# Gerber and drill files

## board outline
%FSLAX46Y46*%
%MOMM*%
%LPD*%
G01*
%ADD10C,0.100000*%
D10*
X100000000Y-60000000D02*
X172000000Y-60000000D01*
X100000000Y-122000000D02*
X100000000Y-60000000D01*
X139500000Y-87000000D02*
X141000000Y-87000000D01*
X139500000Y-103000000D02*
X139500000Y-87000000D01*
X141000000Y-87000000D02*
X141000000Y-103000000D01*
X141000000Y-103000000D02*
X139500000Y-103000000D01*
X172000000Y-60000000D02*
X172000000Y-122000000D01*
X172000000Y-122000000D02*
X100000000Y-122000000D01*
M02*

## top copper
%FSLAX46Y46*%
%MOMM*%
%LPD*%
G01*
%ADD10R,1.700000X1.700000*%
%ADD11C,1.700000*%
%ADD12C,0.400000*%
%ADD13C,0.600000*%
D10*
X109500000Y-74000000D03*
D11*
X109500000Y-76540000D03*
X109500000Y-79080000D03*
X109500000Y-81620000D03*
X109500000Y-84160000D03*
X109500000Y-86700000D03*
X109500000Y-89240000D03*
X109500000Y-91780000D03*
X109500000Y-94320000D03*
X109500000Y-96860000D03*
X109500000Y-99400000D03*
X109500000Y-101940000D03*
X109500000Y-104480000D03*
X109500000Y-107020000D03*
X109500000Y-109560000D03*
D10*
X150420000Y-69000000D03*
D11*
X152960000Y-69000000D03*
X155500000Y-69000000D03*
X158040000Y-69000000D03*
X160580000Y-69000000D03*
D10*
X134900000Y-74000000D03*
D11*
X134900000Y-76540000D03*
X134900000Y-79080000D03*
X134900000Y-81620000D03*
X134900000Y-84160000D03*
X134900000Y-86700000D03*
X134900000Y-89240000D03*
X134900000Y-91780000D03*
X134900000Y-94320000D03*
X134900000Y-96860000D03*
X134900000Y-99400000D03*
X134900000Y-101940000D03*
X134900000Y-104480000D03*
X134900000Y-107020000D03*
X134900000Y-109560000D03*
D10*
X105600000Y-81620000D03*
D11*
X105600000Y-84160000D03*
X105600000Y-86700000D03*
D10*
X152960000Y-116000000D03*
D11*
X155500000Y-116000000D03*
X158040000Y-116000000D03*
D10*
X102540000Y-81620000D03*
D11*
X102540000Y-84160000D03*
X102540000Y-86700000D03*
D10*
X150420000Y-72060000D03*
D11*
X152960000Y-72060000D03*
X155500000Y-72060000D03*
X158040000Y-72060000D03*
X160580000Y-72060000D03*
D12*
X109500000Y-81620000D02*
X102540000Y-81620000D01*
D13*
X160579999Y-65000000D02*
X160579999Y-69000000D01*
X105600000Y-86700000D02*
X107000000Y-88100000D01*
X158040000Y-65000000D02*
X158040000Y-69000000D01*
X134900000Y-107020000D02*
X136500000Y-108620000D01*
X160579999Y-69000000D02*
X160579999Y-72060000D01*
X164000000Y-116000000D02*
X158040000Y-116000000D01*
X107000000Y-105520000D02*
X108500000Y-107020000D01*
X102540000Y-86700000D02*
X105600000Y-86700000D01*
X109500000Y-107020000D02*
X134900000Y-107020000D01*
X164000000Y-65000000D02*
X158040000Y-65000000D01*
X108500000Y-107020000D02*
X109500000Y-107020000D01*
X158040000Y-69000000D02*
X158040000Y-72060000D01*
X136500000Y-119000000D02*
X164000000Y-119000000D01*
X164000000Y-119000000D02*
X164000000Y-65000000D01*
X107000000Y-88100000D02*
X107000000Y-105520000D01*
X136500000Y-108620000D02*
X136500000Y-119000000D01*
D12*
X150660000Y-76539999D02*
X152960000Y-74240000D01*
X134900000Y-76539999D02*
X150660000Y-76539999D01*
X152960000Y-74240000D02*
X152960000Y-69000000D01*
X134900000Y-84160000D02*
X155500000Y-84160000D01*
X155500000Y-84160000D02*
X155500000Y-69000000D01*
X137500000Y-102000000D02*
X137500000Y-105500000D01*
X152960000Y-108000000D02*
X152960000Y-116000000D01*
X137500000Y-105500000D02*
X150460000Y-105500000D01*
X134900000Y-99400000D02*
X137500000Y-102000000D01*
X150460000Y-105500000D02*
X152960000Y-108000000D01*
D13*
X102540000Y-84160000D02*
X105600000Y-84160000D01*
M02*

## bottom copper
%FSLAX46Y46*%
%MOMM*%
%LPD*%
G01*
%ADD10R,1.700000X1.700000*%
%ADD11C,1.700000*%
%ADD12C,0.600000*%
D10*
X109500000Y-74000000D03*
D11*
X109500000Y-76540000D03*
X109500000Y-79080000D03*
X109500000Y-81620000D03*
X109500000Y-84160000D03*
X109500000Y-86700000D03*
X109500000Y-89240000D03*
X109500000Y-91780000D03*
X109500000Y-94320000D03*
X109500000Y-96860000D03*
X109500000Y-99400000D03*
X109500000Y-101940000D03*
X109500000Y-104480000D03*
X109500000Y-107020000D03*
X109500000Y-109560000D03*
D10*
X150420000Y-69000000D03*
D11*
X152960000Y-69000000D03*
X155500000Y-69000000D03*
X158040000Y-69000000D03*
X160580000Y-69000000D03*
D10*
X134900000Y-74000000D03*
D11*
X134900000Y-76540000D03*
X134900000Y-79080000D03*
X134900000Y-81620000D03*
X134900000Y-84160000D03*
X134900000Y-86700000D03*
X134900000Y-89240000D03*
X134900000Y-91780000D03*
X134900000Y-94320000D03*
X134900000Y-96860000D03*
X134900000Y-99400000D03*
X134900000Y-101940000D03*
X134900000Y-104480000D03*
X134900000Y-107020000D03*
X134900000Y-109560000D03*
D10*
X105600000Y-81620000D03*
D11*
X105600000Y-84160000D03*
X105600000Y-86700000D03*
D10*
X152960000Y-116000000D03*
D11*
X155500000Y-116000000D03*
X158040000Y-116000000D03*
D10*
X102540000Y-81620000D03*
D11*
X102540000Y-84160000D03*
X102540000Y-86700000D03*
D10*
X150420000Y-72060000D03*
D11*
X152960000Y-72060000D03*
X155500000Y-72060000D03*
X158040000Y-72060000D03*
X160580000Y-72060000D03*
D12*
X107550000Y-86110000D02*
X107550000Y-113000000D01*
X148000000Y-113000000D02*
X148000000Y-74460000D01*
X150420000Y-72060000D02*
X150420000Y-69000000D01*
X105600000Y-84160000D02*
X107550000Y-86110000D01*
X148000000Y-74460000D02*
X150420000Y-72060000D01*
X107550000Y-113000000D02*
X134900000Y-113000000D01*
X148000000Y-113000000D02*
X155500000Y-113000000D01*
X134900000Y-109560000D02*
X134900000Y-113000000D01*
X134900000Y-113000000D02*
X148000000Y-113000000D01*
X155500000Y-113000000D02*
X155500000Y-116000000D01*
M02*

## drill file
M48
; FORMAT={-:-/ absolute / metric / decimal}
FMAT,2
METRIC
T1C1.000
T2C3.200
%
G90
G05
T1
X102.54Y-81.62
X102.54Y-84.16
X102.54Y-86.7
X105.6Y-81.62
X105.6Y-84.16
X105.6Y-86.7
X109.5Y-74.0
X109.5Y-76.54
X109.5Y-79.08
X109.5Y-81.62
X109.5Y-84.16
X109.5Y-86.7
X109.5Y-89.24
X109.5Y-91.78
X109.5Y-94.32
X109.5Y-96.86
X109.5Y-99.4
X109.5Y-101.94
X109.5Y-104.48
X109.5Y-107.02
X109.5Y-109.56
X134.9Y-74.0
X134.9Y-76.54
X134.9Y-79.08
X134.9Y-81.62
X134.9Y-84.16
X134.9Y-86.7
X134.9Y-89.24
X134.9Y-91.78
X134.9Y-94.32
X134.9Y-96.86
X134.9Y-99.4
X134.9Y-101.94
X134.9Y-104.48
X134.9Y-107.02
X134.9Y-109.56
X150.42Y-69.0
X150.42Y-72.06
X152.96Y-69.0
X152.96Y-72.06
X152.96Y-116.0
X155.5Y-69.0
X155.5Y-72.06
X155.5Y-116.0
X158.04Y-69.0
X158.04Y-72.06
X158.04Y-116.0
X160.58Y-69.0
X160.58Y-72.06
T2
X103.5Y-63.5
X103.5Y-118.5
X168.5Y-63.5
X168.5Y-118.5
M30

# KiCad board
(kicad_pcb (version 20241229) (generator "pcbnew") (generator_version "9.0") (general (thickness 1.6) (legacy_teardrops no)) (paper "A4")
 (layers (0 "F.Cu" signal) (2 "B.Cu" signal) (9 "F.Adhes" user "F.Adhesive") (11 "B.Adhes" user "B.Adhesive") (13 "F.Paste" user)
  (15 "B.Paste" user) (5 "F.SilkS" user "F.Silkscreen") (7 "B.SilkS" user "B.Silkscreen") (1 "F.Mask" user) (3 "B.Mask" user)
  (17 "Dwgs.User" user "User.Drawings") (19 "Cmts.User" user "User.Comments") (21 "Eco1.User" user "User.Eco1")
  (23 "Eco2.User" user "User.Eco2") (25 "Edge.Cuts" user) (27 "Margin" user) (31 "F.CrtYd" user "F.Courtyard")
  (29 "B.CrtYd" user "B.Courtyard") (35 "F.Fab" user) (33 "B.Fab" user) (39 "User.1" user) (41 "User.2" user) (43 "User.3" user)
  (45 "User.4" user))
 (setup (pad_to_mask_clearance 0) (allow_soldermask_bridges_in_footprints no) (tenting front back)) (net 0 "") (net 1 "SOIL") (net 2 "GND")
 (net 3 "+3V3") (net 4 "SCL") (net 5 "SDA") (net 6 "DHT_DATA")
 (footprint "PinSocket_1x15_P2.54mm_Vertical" (layer "F.Cu") (at 109.5 74)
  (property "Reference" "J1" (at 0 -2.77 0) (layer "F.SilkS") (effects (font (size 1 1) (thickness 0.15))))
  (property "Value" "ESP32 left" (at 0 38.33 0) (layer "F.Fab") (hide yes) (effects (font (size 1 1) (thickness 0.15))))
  (pad "1" thru_hole rect (at 0 0) (size 1.7 1.7) (drill 1) (layers "*.Cu" "*.Mask") (remove_unused_layers no))
  (pad "2" thru_hole circle (at 0 2.54) (size 1.7 1.7) (drill 1) (layers "*.Cu" "*.Mask") (remove_unused_layers no))
  (pad "3" thru_hole circle (at 0 5.08) (size 1.7 1.7) (drill 1) (layers "*.Cu" "*.Mask") (remove_unused_layers no))
  (pad "4" thru_hole circle (at 0 7.62) (size 1.7 1.7) (drill 1) (layers "*.Cu" "*.Mask") (remove_unused_layers no) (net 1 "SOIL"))
  (pad "5" thru_hole circle (at 0 10.16) (size 1.7 1.7) (drill 1) (layers "*.Cu" "*.Mask") (remove_unused_layers no))
  (pad "6" thru_hole circle (at 0 12.7) (size 1.7 1.7) (drill 1) (layers "*.Cu" "*.Mask") (remove_unused_layers no))
  (pad "7" thru_hole circle (at 0 15.24) (size 1.7 1.7) (drill 1) (layers "*.Cu" "*.Mask") (remove_unused_layers no))
  (pad "8" thru_hole circle (at 0 17.78) (size 1.7 1.7) (drill 1) (layers "*.Cu" "*.Mask") (remove_unused_layers no))
  (pad "9" thru_hole circle (at 0 20.32) (size 1.7 1.7) (drill 1) (layers "*.Cu" "*.Mask") (remove_unused_layers no))
  (pad "10" thru_hole circle (at 0 22.86) (size 1.7 1.7) (drill 1) (layers "*.Cu" "*.Mask") (remove_unused_layers no))
  (pad "11" thru_hole circle (at 0 25.4) (size 1.7 1.7) (drill 1) (layers "*.Cu" "*.Mask") (remove_unused_layers no))
  (pad "12" thru_hole circle (at 0 27.94) (size 1.7 1.7) (drill 1) (layers "*.Cu" "*.Mask") (remove_unused_layers no))
  (pad "13" thru_hole circle (at 0 30.48) (size 1.7 1.7) (drill 1) (layers "*.Cu" "*.Mask") (remove_unused_layers no))
  (pad "14" thru_hole circle (at 0 33.02) (size 1.7 1.7) (drill 1) (layers "*.Cu" "*.Mask") (remove_unused_layers no) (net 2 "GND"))
  (pad "15" thru_hole circle (at 0 35.56) (size 1.7 1.7) (drill 1) (layers "*.Cu" "*.Mask") (remove_unused_layers no)))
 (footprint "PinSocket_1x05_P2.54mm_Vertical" (layer "F.Cu") (at 150.42 69 90)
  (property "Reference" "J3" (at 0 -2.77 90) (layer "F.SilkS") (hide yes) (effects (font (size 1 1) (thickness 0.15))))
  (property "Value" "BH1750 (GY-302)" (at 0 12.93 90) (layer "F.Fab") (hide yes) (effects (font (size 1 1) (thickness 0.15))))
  (pad "1" thru_hole rect (at 0 0 90) (size 1.7 1.7) (drill 1) (layers "*.Cu" "*.Mask") (remove_unused_layers no) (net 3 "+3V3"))
  (pad "2" thru_hole circle (at 0 2.54 90) (size 1.7 1.7) (drill 1) (layers "*.Cu" "*.Mask") (remove_unused_layers no) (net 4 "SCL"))
  (pad "3" thru_hole circle (at 0 5.08 90) (size 1.7 1.7) (drill 1) (layers "*.Cu" "*.Mask") (remove_unused_layers no) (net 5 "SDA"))
  (pad "4" thru_hole circle (at 0 7.62 90) (size 1.7 1.7) (drill 1) (layers "*.Cu" "*.Mask") (remove_unused_layers no) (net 2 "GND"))
  (pad "5" thru_hole circle (at 0 10.16 90) (size 1.7 1.7) (drill 1) (layers "*.Cu" "*.Mask") (remove_unused_layers no) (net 2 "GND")))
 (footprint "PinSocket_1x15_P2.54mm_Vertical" (layer "F.Cu") (at 134.9 74)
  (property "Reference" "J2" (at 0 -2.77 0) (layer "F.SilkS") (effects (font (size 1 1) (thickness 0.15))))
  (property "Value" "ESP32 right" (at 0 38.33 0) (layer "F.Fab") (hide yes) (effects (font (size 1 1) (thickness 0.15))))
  (pad "1" thru_hole rect (at 0 0) (size 1.7 1.7) (drill 1) (layers "*.Cu" "*.Mask") (remove_unused_layers no))
  (pad "2" thru_hole circle (at 0 2.54) (size 1.7 1.7) (drill 1) (layers "*.Cu" "*.Mask") (remove_unused_layers no) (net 4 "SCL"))
  (pad "3" thru_hole circle (at 0 5.08) (size 1.7 1.7) (drill 1) (layers "*.Cu" "*.Mask") (remove_unused_layers no))
  (pad "4" thru_hole circle (at 0 7.62) (size 1.7 1.7) (drill 1) (layers "*.Cu" "*.Mask") (remove_unused_layers no))
  (pad "5" thru_hole circle (at 0 10.16) (size 1.7 1.7) (drill 1) (layers "*.Cu" "*.Mask") (remove_unused_layers no) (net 5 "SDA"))
  (pad "6" thru_hole circle (at 0 12.7) (size 1.7 1.7) (drill 1) (layers "*.Cu" "*.Mask") (remove_unused_layers no))
  (pad "7" thru_hole circle (at 0 15.24) (size 1.7 1.7) (drill 1) (layers "*.Cu" "*.Mask") (remove_unused_layers no))
  (pad "8" thru_hole circle (at 0 17.78) (size 1.7 1.7) (drill 1) (layers "*.Cu" "*.Mask") (remove_unused_layers no))
  (pad "9" thru_hole circle (at 0 20.32) (size 1.7 1.7) (drill 1) (layers "*.Cu" "*.Mask") (remove_unused_layers no))
  (pad "10" thru_hole circle (at 0 22.86) (size 1.7 1.7) (drill 1) (layers "*.Cu" "*.Mask") (remove_unused_layers no))
  (pad "11" thru_hole circle (at 0 25.4) (size 1.7 1.7) (drill 1) (layers "*.Cu" "*.Mask") (remove_unused_layers no) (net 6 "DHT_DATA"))
  (pad "12" thru_hole circle (at 0 27.94) (size 1.7 1.7) (drill 1) (layers "*.Cu" "*.Mask") (remove_unused_layers no))
  (pad "13" thru_hole circle (at 0 30.48) (size 1.7 1.7) (drill 1) (layers "*.Cu" "*.Mask") (remove_unused_layers no))
  (pad "14" thru_hole circle (at 0 33.02) (size 1.7 1.7) (drill 1) (layers "*.Cu" "*.Mask") (remove_unused_layers no) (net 2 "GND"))
  (pad "15" thru_hole circle (at 0 35.56) (size 1.7 1.7) (drill 1) (layers "*.Cu" "*.Mask") (remove_unused_layers no) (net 3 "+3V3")))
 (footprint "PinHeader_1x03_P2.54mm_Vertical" (layer "F.Cu") (at 105.6 81.62)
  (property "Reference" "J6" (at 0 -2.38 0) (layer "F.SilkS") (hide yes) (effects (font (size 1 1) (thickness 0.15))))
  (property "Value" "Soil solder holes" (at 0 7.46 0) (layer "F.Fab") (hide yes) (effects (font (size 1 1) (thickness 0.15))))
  (pad "1" thru_hole rect (at 0 0) (size 1.7 1.7) (drill 1) (layers "*.Cu" "*.Mask") (remove_unused_layers no) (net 1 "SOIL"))
  (pad "2" thru_hole circle (at 0 2.54) (size 1.7 1.7) (drill 1) (layers "*.Cu" "*.Mask") (remove_unused_layers no) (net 3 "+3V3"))
  (pad "3" thru_hole circle (at 0 5.08) (size 1.7 1.7) (drill 1) (layers "*.Cu" "*.Mask") (remove_unused_layers no) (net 2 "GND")))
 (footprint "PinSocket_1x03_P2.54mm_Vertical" (layer "F.Cu") (at 152.96 116 90)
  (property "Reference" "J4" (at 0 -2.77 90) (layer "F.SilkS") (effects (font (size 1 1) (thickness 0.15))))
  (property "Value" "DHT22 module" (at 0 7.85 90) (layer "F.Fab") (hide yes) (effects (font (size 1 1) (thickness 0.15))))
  (pad "1" thru_hole rect (at 0 0 90) (size 1.7 1.7) (drill 1) (layers "*.Cu" "*.Mask") (remove_unused_layers no) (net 6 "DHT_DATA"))
  (pad "2" thru_hole circle (at 0 2.54 90) (size 1.7 1.7) (drill 1) (layers "*.Cu" "*.Mask") (remove_unused_layers no) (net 3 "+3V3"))
  (pad "3" thru_hole circle (at 0 5.08 90) (size 1.7 1.7) (drill 1) (layers "*.Cu" "*.Mask") (remove_unused_layers no) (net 2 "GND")))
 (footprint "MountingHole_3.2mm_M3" (layer "F.Cu") (at 103.5 118.5)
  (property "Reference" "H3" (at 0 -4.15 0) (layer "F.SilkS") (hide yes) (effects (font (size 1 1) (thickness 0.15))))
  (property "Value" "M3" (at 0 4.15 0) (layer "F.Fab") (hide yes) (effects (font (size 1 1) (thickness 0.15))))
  (pad "" np_thru_hole circle (at 0 0) (size 3.2 3.2) (drill 3.2) (layers "*.Cu" "*.Mask")))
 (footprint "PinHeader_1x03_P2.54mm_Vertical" (layer "F.Cu") (at 102.54 81.62)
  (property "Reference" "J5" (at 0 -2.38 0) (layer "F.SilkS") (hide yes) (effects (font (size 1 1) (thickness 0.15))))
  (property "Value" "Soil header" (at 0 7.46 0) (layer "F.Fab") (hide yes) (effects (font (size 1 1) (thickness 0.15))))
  (pad "1" thru_hole rect (at 0 0) (size 1.7 1.7) (drill 1) (layers "*.Cu" "*.Mask") (remove_unused_layers no) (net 1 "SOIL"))
  (pad "2" thru_hole circle (at 0 2.54) (size 1.7 1.7) (drill 1) (layers "*.Cu" "*.Mask") (remove_unused_layers no) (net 3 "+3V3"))
  (pad "3" thru_hole circle (at 0 5.08) (size 1.7 1.7) (drill 1) (layers "*.Cu" "*.Mask") (remove_unused_layers no) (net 2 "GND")))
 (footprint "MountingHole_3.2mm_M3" (layer "F.Cu") (at 168.5 118.5)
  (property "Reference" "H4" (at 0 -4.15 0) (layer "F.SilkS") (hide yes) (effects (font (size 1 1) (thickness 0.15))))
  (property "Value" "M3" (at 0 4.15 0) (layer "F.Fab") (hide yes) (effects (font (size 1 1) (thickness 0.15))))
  (pad "" np_thru_hole circle (at 0 0) (size 3.2 3.2) (drill 3.2) (layers "*.Cu" "*.Mask")))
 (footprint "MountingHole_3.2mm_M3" (layer "F.Cu") (at 168.5 63.5)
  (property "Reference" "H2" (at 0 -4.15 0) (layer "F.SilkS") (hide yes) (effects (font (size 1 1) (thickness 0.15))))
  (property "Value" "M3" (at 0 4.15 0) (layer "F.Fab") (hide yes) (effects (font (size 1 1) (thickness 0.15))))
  (pad "" np_thru_hole circle (at 0 0) (size 3.2 3.2) (drill 3.2) (layers "*.Cu" "*.Mask")))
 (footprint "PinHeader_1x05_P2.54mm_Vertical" (layer "F.Cu") (at 150.42 72.06 90)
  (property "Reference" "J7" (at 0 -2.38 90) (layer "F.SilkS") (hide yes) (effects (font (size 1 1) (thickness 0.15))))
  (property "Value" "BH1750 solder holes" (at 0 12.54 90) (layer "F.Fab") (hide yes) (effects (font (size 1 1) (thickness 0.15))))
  (pad "1" thru_hole rect (at 0 0 90) (size 1.7 1.7) (drill 1) (layers "*.Cu" "*.Mask") (remove_unused_layers no) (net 3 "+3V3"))
  (pad "2" thru_hole circle (at 0 2.54 90) (size 1.7 1.7) (drill 1) (layers "*.Cu" "*.Mask") (remove_unused_layers no) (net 4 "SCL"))
  (pad "3" thru_hole circle (at 0 5.08 90) (size 1.7 1.7) (drill 1) (layers "*.Cu" "*.Mask") (remove_unused_layers no) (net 5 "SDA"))
  (pad "4" thru_hole circle (at 0 7.62 90) (size 1.7 1.7) (drill 1) (layers "*.Cu" "*.Mask") (remove_unused_layers no) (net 2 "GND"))
  (pad "5" thru_hole circle (at 0 10.16 90) (size 1.7 1.7) (drill 1) (layers "*.Cu" "*.Mask") (remove_unused_layers no) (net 2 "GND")))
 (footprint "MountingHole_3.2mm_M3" (layer "F.Cu") (at 103.5 63.5)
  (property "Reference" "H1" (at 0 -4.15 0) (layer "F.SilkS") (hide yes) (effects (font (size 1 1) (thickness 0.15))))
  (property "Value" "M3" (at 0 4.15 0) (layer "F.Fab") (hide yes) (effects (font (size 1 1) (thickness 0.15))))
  (pad "" np_thru_hole circle (at 0 0) (size 3.2 3.2) (drill 3.2) (layers "*.Cu" "*.Mask")))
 (gr_line (start 100 60) (end 172 60) (stroke (width 0.1) (type default)) (layer "Edge.Cuts"))
 (gr_line (start 100 122) (end 100 60) (stroke (width 0.1) (type default)) (layer "Edge.Cuts"))
 (gr_line (start 139.5 87) (end 141 87) (stroke (width 0.1) (type default)) (layer "Edge.Cuts"))
 (gr_line (start 139.5 103) (end 139.5 87) (stroke (width 0.1) (type default)) (layer "Edge.Cuts"))
 (gr_line (start 141 87) (end 141 103) (stroke (width 0.1) (type default)) (layer "Edge.Cuts"))
 (gr_line (start 141 103) (end 139.5 103) (stroke (width 0.1) (type default)) (layer "Edge.Cuts"))
 (gr_line (start 172 60) (end 172 122) (stroke (width 0.1) (type default)) (layer "Edge.Cuts"))
 (gr_line (start 172 122) (end 100 122) (stroke (width 0.1) (type default)) (layer "Edge.Cuts"))
 (segment (start 109.5 81.62) (end 102.54 81.62) (width 0.4) (layer "F.Cu") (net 1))
 (segment (start 160.579999 65) (end 160.579999 69) (width 0.6) (layer "F.Cu") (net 2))
 (segment (start 105.6 86.7) (end 107 88.1) (width 0.6) (layer "F.Cu") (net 2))
 (segment (start 158.04 65) (end 158.04 69) (width 0.6) (layer "F.Cu") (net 2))
 (segment (start 134.9 107.02) (end 136.5 108.62) (width 0.6) (layer "F.Cu") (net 2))
 (segment (start 160.579999 69) (end 160.579999 72.06) (width 0.6) (layer "F.Cu") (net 2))
 (segment (start 164 116) (end 158.04 116) (width 0.6) (layer "F.Cu") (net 2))
 (segment (start 107 105.52) (end 108.5 107.02) (width 0.6) (layer "F.Cu") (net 2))
 (segment (start 102.54 86.7) (end 105.6 86.7) (width 0.6) (layer "F.Cu") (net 2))
 (segment (start 109.5 107.02) (end 134.9 107.02) (width 0.6) (layer "F.Cu") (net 2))
 (segment (start 164 65) (end 158.04 65) (width 0.6) (layer "F.Cu") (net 2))
 (segment (start 108.5 107.02) (end 109.5 107.02) (width 0.6) (layer "F.Cu") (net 2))
 (segment (start 158.04 69) (end 158.04 72.06) (width 0.6) (layer "F.Cu") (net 2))
 (segment (start 136.5 119) (end 164 119) (width 0.6) (layer "F.Cu") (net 2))
 (segment (start 164 119) (end 164 65) (width 0.6) (layer "F.Cu") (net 2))
 (segment (start 107 88.1) (end 107 105.52) (width 0.6) (layer "F.Cu") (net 2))
 (segment (start 136.5 108.62) (end 136.5 119) (width 0.6) (layer "F.Cu") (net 2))
 (segment (start 150.66 76.539999) (end 152.96 74.24) (width 0.4) (layer "F.Cu") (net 4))
 (segment (start 134.9 76.539999) (end 150.66 76.539999) (width 0.4) (layer "F.Cu") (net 4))
 (segment (start 152.96 74.24) (end 152.96 69) (width 0.4) (layer "F.Cu") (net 4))
 (segment (start 134.9 84.16) (end 155.5 84.16) (width 0.4) (layer "F.Cu") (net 5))
 (segment (start 155.5 84.16) (end 155.5 69) (width 0.4) (layer "F.Cu") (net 5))
 (segment (start 137.5 102) (end 137.5 105.5) (width 0.4) (layer "F.Cu") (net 6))
 (segment (start 152.96 108) (end 152.96 116) (width 0.4) (layer "F.Cu") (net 6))
 (segment (start 137.5 105.5) (end 150.46 105.5) (width 0.4) (layer "F.Cu") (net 6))
 (segment (start 134.9 99.4) (end 137.5 102) (width 0.4) (layer "F.Cu") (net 6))
 (segment (start 150.46 105.5) (end 152.96 108) (width 0.4) (layer "F.Cu") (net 6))
 (segment (start 102.54 84.16) (end 105.6 84.16) (width 0.6) (layer "F.Cu") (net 3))
 (segment (start 107.55 86.11) (end 107.55 113) (width 0.6) (layer "B.Cu") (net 3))
 (segment (start 148 113) (end 148 74.46) (width 0.6) (layer "B.Cu") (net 3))
 (segment (start 150.42 72.06) (end 150.42 69) (width 0.6) (layer "B.Cu") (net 3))
 (segment (start 105.6 84.16) (end 107.55 86.11) (width 0.6) (layer "B.Cu") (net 3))
 (segment (start 148 74.46) (end 150.42 72.06) (width 0.6) (layer "B.Cu") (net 3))
 (segment (start 107.55 113) (end 134.9 113) (width 0.6) (layer "B.Cu") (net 3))
 (segment (start 148 113) (end 155.5 113) (width 0.6) (layer "B.Cu") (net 3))
 (segment (start 134.9 109.56) (end 134.9 113) (width 0.6) (layer "B.Cu") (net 3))
 (segment (start 134.9 113) (end 148 113) (width 0.6) (layer "B.Cu") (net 3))
 (segment (start 155.5 113) (end 155.5 116) (width 0.6) (layer "B.Cu") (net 3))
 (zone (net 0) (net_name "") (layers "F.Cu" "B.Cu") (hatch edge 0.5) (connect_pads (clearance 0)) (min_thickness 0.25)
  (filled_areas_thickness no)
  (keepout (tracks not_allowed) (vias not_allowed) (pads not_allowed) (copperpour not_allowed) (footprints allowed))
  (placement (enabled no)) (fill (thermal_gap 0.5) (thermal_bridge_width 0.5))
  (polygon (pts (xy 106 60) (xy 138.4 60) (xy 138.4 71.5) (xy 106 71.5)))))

